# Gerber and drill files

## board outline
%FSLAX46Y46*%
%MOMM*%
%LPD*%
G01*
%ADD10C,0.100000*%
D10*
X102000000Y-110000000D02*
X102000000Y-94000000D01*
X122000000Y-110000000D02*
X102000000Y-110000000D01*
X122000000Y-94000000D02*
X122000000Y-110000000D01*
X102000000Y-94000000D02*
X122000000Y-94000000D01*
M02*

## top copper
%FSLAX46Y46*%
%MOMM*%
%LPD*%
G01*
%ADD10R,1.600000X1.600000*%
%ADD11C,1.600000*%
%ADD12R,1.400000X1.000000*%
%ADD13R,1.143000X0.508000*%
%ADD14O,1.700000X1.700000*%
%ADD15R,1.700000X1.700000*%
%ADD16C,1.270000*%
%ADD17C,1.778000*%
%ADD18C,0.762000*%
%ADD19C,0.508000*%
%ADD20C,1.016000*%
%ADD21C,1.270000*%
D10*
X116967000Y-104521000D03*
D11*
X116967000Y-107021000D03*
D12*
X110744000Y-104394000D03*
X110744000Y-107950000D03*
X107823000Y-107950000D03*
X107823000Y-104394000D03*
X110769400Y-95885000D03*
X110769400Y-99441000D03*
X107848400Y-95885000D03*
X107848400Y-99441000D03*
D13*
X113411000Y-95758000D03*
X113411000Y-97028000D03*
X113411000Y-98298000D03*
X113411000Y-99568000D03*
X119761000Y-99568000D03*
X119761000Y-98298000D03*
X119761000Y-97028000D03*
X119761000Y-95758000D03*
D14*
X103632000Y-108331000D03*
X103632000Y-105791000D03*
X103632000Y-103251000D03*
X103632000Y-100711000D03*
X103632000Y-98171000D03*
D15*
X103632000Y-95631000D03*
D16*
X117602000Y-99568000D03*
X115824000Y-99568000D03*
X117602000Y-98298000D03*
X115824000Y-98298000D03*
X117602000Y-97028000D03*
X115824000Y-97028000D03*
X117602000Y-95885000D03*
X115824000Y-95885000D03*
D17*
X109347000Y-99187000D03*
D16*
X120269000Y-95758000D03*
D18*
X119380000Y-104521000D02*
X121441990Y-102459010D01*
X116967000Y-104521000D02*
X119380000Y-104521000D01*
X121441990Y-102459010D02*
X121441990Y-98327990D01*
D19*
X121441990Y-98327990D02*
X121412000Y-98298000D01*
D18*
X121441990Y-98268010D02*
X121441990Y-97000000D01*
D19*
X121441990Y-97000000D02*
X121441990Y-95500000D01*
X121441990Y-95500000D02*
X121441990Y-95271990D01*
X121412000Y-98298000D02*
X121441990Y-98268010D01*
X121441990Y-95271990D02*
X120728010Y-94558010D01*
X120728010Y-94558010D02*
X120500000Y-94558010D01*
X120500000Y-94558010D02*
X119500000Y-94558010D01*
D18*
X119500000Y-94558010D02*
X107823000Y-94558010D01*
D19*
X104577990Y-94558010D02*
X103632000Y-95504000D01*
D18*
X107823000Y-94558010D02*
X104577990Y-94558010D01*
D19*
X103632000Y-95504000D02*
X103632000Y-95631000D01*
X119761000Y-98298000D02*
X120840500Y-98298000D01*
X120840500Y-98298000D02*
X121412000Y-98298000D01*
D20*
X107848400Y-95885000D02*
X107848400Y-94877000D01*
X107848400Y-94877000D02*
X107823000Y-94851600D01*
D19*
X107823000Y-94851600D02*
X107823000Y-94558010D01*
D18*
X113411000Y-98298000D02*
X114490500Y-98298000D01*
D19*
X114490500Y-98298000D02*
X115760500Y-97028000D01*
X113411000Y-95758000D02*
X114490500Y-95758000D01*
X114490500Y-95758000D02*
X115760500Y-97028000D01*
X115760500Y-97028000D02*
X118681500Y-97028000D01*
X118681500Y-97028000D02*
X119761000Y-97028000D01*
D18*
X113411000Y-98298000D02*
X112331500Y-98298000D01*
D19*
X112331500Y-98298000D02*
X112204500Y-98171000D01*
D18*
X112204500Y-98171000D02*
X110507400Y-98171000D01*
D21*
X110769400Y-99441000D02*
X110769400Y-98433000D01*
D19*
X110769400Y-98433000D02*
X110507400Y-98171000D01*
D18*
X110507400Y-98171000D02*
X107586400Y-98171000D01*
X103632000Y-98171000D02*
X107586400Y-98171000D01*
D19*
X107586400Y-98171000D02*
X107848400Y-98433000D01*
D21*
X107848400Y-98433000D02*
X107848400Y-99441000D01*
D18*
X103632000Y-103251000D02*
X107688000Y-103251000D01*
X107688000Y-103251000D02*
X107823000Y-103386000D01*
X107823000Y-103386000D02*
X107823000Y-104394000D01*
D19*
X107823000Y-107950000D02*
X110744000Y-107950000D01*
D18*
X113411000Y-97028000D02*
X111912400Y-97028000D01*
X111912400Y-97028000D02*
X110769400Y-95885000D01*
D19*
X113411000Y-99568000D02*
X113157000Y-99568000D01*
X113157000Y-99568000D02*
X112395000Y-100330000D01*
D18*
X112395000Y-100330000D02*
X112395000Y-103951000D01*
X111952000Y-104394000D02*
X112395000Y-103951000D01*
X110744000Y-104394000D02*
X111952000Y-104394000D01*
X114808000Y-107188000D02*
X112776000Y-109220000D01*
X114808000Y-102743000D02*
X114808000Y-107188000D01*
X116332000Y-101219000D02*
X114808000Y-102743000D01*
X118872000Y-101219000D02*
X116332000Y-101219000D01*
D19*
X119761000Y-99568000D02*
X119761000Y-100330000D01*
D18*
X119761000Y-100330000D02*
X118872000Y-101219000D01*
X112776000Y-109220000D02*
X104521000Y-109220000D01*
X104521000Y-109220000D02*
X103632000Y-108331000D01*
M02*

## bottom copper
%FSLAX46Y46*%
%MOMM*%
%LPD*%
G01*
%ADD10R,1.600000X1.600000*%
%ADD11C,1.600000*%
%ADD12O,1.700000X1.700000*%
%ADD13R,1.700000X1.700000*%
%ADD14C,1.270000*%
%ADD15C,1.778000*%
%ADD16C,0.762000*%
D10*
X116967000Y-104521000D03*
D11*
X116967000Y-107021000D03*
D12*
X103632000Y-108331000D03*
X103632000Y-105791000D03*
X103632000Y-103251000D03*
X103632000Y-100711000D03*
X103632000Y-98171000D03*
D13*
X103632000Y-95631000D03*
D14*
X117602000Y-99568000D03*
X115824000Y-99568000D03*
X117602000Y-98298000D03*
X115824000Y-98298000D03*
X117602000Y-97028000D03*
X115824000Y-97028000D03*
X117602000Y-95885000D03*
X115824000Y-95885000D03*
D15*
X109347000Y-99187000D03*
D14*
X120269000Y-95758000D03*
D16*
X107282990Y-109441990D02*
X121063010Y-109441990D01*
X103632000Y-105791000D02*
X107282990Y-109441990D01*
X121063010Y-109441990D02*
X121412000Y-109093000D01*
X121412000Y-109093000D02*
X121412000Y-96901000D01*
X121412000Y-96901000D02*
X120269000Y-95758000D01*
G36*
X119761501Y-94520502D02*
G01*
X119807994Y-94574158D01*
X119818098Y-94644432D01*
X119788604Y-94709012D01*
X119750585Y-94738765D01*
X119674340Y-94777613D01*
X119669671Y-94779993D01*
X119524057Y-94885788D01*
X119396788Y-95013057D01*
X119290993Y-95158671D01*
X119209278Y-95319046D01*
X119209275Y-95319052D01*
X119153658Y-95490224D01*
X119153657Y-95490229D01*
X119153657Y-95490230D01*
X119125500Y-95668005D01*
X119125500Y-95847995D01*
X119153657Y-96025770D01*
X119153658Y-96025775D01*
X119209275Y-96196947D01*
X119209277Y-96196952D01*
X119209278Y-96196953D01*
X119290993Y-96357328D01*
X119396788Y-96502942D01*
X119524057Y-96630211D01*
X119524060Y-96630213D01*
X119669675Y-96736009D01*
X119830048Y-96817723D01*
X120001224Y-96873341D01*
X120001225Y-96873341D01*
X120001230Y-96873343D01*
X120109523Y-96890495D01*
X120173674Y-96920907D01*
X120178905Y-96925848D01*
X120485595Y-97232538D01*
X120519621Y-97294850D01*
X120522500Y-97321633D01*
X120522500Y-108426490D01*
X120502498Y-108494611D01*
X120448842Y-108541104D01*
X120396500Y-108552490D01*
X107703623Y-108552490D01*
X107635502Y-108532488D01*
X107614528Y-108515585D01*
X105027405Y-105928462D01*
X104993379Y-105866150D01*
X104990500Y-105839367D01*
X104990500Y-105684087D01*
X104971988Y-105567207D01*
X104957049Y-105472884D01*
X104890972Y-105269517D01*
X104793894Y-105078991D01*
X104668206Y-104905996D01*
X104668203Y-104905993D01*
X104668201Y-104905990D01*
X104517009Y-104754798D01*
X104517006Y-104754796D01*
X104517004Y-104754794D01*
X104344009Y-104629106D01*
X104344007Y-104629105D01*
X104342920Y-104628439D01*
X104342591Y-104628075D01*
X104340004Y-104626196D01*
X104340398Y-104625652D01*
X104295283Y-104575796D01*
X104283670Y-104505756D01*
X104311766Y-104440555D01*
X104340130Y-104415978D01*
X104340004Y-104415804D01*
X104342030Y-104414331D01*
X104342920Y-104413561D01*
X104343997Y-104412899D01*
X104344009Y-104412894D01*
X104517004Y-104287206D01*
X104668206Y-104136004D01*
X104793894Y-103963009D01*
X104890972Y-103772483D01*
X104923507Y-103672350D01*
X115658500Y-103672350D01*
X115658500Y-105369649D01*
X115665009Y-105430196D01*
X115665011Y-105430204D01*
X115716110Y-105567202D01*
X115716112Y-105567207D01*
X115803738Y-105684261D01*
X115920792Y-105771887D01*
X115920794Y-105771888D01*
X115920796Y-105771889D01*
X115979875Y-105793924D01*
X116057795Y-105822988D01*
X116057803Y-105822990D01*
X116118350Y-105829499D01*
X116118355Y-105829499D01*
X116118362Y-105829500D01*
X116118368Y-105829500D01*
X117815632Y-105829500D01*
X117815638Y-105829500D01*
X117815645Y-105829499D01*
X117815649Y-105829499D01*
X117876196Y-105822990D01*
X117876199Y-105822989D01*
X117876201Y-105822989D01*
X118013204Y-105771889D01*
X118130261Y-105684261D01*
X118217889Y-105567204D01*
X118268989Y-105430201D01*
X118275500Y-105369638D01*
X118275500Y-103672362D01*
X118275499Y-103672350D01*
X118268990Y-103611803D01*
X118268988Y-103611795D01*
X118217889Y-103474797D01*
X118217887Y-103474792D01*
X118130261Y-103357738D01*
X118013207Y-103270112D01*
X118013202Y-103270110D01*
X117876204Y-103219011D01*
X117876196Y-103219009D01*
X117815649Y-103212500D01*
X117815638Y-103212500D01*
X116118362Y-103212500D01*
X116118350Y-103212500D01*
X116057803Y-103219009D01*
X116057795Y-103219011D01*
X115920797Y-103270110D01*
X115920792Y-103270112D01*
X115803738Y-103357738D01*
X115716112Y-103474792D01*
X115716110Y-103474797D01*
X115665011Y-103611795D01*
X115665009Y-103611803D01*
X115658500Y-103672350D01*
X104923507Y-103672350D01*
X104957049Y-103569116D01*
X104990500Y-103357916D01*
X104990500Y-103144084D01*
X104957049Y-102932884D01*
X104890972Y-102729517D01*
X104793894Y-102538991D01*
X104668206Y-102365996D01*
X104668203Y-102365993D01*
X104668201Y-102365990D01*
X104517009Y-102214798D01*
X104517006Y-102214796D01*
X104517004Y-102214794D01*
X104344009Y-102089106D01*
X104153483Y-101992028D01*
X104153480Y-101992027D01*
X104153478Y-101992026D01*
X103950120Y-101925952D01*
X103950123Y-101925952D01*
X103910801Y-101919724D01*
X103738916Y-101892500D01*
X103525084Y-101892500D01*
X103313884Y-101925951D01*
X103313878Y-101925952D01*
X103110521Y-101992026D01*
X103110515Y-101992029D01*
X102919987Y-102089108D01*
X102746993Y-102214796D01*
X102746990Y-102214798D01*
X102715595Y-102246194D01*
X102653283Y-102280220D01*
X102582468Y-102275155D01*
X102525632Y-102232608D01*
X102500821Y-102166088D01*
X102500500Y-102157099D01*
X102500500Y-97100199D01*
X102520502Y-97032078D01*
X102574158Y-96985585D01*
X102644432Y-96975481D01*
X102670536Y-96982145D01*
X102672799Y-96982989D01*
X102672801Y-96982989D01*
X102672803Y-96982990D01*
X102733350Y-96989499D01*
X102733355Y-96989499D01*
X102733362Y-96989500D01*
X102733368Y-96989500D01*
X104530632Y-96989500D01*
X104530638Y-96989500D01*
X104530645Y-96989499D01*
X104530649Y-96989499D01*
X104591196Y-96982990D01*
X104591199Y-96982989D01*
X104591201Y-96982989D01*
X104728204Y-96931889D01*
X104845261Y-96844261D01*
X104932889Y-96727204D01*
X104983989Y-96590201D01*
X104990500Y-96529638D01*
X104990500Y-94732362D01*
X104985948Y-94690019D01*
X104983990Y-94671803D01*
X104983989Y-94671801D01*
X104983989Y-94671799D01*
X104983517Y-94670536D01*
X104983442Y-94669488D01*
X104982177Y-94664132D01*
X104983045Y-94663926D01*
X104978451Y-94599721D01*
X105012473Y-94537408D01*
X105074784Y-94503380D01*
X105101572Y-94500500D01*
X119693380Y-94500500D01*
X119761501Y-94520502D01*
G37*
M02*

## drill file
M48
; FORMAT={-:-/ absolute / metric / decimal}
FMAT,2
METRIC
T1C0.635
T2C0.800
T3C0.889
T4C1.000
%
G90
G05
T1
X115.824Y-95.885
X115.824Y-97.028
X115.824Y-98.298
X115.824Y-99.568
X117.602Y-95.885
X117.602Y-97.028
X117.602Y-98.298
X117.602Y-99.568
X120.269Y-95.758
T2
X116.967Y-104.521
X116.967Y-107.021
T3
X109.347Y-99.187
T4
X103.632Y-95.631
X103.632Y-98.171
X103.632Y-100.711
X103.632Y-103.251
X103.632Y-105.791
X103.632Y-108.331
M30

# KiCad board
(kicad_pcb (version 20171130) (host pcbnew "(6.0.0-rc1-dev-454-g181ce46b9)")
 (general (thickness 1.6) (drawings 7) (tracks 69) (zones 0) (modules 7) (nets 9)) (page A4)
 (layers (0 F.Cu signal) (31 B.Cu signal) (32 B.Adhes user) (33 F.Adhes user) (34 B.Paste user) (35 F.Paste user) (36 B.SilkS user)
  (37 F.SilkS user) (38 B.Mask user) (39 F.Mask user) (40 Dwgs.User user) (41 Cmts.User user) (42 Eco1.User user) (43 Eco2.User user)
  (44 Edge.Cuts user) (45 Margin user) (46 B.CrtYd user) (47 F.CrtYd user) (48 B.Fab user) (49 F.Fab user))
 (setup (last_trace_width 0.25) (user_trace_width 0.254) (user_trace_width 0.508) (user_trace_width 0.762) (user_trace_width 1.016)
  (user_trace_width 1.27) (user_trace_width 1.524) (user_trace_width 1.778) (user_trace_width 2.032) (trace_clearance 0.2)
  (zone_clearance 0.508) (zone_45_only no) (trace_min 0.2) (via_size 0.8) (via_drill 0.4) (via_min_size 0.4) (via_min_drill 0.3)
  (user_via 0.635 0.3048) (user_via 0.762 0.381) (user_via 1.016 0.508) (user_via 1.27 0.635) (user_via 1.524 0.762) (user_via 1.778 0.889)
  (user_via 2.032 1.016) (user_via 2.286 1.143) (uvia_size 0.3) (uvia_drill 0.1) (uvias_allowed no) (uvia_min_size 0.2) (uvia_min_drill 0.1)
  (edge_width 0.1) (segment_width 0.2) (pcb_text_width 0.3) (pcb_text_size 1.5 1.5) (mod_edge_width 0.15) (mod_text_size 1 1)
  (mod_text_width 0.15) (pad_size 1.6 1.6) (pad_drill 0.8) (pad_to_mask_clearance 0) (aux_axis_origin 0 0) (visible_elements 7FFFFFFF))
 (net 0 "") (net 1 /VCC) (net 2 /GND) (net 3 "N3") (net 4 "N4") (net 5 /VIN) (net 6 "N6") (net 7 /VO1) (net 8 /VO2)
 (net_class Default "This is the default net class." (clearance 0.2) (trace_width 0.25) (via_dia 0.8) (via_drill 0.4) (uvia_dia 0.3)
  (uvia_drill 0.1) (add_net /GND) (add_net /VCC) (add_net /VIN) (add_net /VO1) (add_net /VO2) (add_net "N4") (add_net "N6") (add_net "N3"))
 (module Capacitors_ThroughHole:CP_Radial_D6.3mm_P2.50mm (layer F.Cu) (at 116.967 104.521 270)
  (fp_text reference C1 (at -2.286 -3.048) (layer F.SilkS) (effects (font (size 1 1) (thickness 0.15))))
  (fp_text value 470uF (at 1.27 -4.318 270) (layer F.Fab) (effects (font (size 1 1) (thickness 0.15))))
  (pad 1 thru_hole rect (at 0 0 270) (size 1.6 1.6) (drill 0.8) (layers *.Cu *.Mask) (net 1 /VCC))
  (pad 2 thru_hole circle (at 2.5 0 270) (size 1.6 1.6) (drill 0.8) (layers *.Cu *.Mask) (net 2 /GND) (zone_connect 2)))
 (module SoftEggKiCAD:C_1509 (layer F.Cu) (at 110.5916 105.918 270)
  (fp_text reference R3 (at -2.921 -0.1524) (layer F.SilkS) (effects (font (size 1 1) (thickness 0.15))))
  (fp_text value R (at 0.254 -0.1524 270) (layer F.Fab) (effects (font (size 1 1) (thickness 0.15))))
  (pad 1 smd rect (at -1.524 -0.1524 270) (size 1 1.4) (layers F.Cu F.Paste F.Mask) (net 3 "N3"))
  (pad 2 smd rect (at 2.032 -0.1524 270) (size 1 1.4) (layers F.Cu F.Paste F.Mask) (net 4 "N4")))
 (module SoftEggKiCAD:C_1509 (layer F.Cu) (at 107.9754 106.426 90)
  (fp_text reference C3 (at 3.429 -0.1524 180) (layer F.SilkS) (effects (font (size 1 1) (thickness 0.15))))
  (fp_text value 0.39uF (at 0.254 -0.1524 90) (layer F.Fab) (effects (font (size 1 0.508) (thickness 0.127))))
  (pad 1 smd rect (at -1.524 -0.1524 90) (size 1 1.4) (layers F.Cu F.Paste F.Mask) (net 4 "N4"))
  (pad 2 smd rect (at 2.032 -0.1524 90) (size 1 1.4) (layers F.Cu F.Paste F.Mask) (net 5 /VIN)))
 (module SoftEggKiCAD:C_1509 (layer F.Cu) (at 110.617 97.409 270)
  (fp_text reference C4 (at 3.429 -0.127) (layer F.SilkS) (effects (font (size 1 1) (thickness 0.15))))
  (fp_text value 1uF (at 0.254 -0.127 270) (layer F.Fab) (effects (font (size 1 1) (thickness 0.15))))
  (pad 1 smd rect (at -1.524 -0.1524 270) (size 1 1.4) (layers F.Cu F.Paste F.Mask) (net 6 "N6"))
  (pad 2 smd rect (at 2.032 -0.1524 270) (size 1 1.4) (layers F.Cu F.Paste F.Mask) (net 2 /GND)))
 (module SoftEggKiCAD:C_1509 (layer F.Cu) (at 107.696 97.409 270)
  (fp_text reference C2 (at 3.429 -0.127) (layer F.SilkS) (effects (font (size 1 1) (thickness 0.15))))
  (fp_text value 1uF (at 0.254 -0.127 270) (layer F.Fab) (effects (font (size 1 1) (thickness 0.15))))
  (pad 1 smd rect (at -1.524 -0.1524 270) (size 1 1.4) (layers F.Cu F.Paste F.Mask) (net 1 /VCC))
  (pad 2 smd rect (at 2.032 -0.1524 270) (size 1 1.4) (layers F.Cu F.Paste F.Mask) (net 2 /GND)))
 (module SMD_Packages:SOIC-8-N (layer F.Cu) (at 116.586 97.663 270)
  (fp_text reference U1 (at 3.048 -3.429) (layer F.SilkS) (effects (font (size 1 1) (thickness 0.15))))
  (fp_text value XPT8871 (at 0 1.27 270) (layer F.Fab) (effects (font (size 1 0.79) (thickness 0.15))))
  (pad 1 smd rect (at -1.905 3.175 270) (size 0.508 1.143) (layers F.Cu F.Paste F.Mask) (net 2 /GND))
  (pad 2 smd rect (at -0.635 3.175 270) (size 0.508 1.143) (layers F.Cu F.Paste F.Mask) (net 6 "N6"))
  (pad 3 smd rect (at 0.635 3.175 270) (size 0.508 1.143) (layers F.Cu F.Paste F.Mask) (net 2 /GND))
  (pad 4 smd rect (at 1.905 3.175 270) (size 0.508 1.143) (layers F.Cu F.Paste F.Mask) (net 3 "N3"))
  (pad 5 smd rect (at 1.905 -3.175 270) (size 0.508 1.143) (layers F.Cu F.Paste F.Mask) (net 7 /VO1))
  (pad 6 smd rect (at 0.635 -3.175 270) (size 0.508 1.143) (layers F.Cu F.Paste F.Mask) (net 1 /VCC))
  (pad 7 smd rect (at -0.635 -3.175 270) (size 0.508 1.143) (layers F.Cu F.Paste F.Mask) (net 2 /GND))
  (pad 8 smd rect (at -1.905 -3.175 270) (size 0.508 1.143) (layers F.Cu F.Paste F.Mask) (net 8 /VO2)))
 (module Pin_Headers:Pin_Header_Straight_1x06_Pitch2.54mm (layer F.Cu) (at 103.632 95.631)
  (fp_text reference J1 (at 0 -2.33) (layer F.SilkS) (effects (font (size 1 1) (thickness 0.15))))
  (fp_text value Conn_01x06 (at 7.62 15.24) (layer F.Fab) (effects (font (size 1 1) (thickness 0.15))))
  (pad 6 thru_hole oval (at 0 12.7) (size 1.7 1.7) (drill 1) (layers *.Cu *.Mask) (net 7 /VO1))
  (pad 5 thru_hole oval (at 0 10.16) (size 1.7 1.7) (drill 1) (layers *.Cu *.Mask) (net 8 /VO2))
  (pad 4 thru_hole oval (at 0 7.62) (size 1.7 1.7) (drill 1) (layers *.Cu *.Mask) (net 5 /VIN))
  (pad 3 thru_hole oval (at 0 5.08) (size 1.7 1.7) (drill 1) (layers *.Cu *.Mask) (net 2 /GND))
  (pad 2 thru_hole oval (at 0 2.54) (size 1.7 1.7) (drill 1) (layers *.Cu *.Mask) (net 2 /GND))
  (pad 1 thru_hole rect (at 0 0) (size 1.7 1.7) (drill 1) (layers *.Cu *.Mask) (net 1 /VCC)))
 (gr_line (start 102 110) (end 102 94) (layer Edge.Cuts) (width 0.1))
 (gr_line (start 122 110) (end 102 110) (layer Edge.Cuts) (width 0.1))
 (gr_line (start 122 94) (end 122 110) (layer Edge.Cuts) (width 0.1))
 (gr_line (start 102 94) (end 122 94) (layer Edge.Cuts) (width 0.1))
 (segment (start 119.38 104.521) (end 121.44199 102.45901) (width 0.762) (layer F.Cu) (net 1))
 (segment (start 116.967 104.521) (end 119.38 104.521) (width 0.762) (layer F.Cu) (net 1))
 (segment (start 121.44199 102.45901) (end 121.44199 98.32799) (width 0.762) (layer F.Cu) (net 1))
 (segment (start 121.44199 98.32799) (end 121.412 98.298) (width 0.508) (layer F.Cu) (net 1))
 (segment (start 121.44199 98.26801) (end 121.44199 97) (width 0.762) (layer F.Cu) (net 1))
 (segment (start 121.44199 97) (end 121.44199 95.5) (width 0.508) (layer F.Cu) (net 1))
 (segment (start 121.44199 95.5) (end 121.44199 95.27199) (width 0.508) (layer F.Cu) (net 1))
 (segment (start 121.412 98.298) (end 121.44199 98.26801) (width 0.508) (layer F.Cu) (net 1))
 (segment (start 121.44199 95.27199) (end 120.72801 94.55801) (width 0.508) (layer F.Cu) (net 1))
 (segment (start 120.72801 94.55801) (end 120.5 94.55801) (width 0.508) (layer F.Cu) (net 1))
 (segment (start 120.5 94.55801) (end 119.5 94.55801) (width 0.508) (layer F.Cu) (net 1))
 (segment (start 119.5 94.55801) (end 107.823 94.55801) (width 0.762) (layer F.Cu) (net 1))
 (segment (start 104.57799 94.55801) (end 103.632 95.504) (width 0.508) (layer F.Cu) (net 1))
 (segment (start 107.823 94.55801) (end 104.57799 94.55801) (width 0.762) (layer F.Cu) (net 1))
 (segment (start 103.632 95.504) (end 103.632 95.631) (width 0.508) (layer F.Cu) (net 1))
 (segment (start 119.761 98.298) (end 120.8405 98.298) (width 0.508) (layer F.Cu) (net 1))
 (segment (start 120.8405 98.298) (end 121.412 98.298) (width 0.508) (layer F.Cu) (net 1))
 (segment (start 107.8484 95.885) (end 107.8484 94.877) (width 1.016) (layer F.Cu) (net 1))
 (segment (start 107.8484 94.877) (end 107.823 94.8516) (width 1.016) (layer F.Cu) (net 1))
 (segment (start 107.823 94.8516) (end 107.823 94.55801) (width 0.508) (layer F.Cu) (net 1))
 (via (at 117.602 99.568) (size 1.27) (drill 0.635) (layers F.Cu B.Cu) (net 2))
 (via (at 115.824 99.568) (size 1.27) (drill 0.635) (layers F.Cu B.Cu) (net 2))
 (via (at 117.602 98.298) (size 1.27) (drill 0.635) (layers F.Cu B.Cu) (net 2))
 (via (at 115.824 98.298) (size 1.27) (drill 0.635) (layers F.Cu B.Cu) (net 2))
 (via (at 117.602 97.028) (size 1.27) (drill 0.635) (layers F.Cu B.Cu) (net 2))
 (via (at 115.824 97.028) (size 1.27) (drill 0.635) (layers F.Cu B.Cu) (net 2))
 (via (at 117.602 95.885) (size 1.27) (drill 0.635) (layers F.Cu B.Cu) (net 2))
 (via (at 115.824 95.885) (size 1.27) (drill 0.635) (layers F.Cu B.Cu) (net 2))
 (via (at 109.347 99.187) (size 1.778) (drill 0.889) (layers F.Cu B.Cu) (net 2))
 (segment (start 113.411 98.298) (end 114.4905 98.298) (width 0.762) (layer F.Cu) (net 2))
 (segment (start 114.4905 98.298) (end 115.7605 97.028) (width 0.508) (layer F.Cu) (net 2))
 (segment (start 113.411 95.758) (end 114.4905 95.758) (width 0.508) (layer F.Cu) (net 2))
 (segment (start 114.4905 95.758) (end 115.7605 97.028) (width 0.508) (layer F.Cu) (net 2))
 (segment (start 115.7605 97.028) (end 118.6815 97.028) (width 0.508) (layer F.Cu) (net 2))
 (segment (start 118.6815 97.028) (end 119.761 97.028) (width 0.508) (layer F.Cu) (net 2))
 (segment (start 113.411 98.298) (end 112.3315 98.298) (width 0.762) (layer F.Cu) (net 2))
 (segment (start 112.3315 98.298) (end 112.2045 98.171) (width 0.508) (layer F.Cu) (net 2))
 (segment (start 112.2045 98.171) (end 110.5074 98.171) (width 0.762) (layer F.Cu) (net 2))
 (segment (start 110.7694 99.441) (end 110.7694 98.433) (width 1.27) (layer F.Cu) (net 2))
 (segment (start 110.7694 98.433) (end 110.5074 98.171) (width 0.508) (layer F.Cu) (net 2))
 (segment (start 110.5074 98.171) (end 107.5864 98.171) (width 0.762) (layer F.Cu) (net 2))
 (segment (start 103.632 98.171) (end 107.5864 98.171) (width 0.762) (layer F.Cu) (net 2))
 (segment (start 107.5864 98.171) (end 107.8484 98.433) (width 0.508) (layer F.Cu) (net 2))
 (segment (start 107.8484 98.433) (end 107.8484 99.441) (width 1.27) (layer F.Cu) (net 2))
 (segment (start 103.632 103.251) (end 107.688 103.251) (width 0.762) (layer F.Cu) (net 5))
 (segment (start 107.688 103.251) (end 107.823 103.386) (width 0.762) (layer F.Cu) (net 5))
 (segment (start 107.823 103.386) (end 107.823 104.394) (width 0.762) (layer F.Cu) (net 5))
 (segment (start 107.823 107.95) (end 110.744 107.95) (width 0.508) (layer F.Cu) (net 4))
 (segment (start 113.411 97.028) (end 111.9124 97.028) (width 0.762) (layer F.Cu) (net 6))
 (segment (start 111.9124 97.028) (end 110.7694 95.885) (width 0.762) (layer F.Cu) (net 6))
 (segment (start 113.411 99.568) (end 113.157 99.568) (width 0.508) (layer F.Cu) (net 3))
 (segment (start 113.157 99.568) (end 112.395 100.33) (width 0.508) (layer F.Cu) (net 3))
 (segment (start 112.395 100.33) (end 112.395 103.951) (width 0.762) (layer F.Cu) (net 3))
 (segment (start 111.952 104.394) (end 112.395 103.951) (width 0.762) (layer F.Cu) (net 3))
 (segment (start 110.744 104.394) (end 111.952 104.394) (width 0.762) (layer F.Cu) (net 3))
 (segment (start 114.808 107.188) (end 112.776 109.22) (width 0.762) (layer F.Cu) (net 7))
 (segment (start 114.808 102.743) (end 114.808 107.188) (width 0.762) (layer F.Cu) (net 7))
 (segment (start 116.332 101.219) (end 114.808 102.743) (width 0.762) (layer F.Cu) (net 7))
 (segment (start 118.872 101.219) (end 116.332 101.219) (width 0.762) (layer F.Cu) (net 7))
 (segment (start 119.761 99.568) (end 119.761 100.33) (width 0.508) (layer F.Cu) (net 7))
 (segment (start 119.761 100.33) (end 118.872 101.219) (width 0.762) (layer F.Cu) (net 7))
 (segment (start 112.776 109.22) (end 104.521 109.22) (width 0.762) (layer F.Cu) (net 7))
 (segment (start 104.521 109.22) (end 103.632 108.331) (width 0.762) (layer F.Cu) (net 7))
 (segment (start 107.28299 109.44199) (end 121.06301 109.44199) (width 0.762) (layer B.Cu) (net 8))
 (segment (start 103.632 105.791) (end 107.28299 109.44199) (width 0.762) (layer B.Cu) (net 8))
 (segment (start 121.06301 109.44199) (end 121.412 109.093) (width 0.762) (layer B.Cu) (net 8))
 (segment (start 121.412 109.093) (end 121.412 96.901) (width 0.762) (layer B.Cu) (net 8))
 (segment (start 121.412 96.901) (end 120.269 95.758) (width 0.762) (layer B.Cu) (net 8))
 (via (at 120.269 95.758) (size 1.27) (drill 0.635) (layers F.Cu B.Cu) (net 8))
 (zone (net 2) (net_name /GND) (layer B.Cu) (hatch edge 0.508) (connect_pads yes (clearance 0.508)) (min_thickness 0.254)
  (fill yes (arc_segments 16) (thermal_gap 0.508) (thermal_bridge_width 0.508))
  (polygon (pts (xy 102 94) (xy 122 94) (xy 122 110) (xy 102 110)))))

